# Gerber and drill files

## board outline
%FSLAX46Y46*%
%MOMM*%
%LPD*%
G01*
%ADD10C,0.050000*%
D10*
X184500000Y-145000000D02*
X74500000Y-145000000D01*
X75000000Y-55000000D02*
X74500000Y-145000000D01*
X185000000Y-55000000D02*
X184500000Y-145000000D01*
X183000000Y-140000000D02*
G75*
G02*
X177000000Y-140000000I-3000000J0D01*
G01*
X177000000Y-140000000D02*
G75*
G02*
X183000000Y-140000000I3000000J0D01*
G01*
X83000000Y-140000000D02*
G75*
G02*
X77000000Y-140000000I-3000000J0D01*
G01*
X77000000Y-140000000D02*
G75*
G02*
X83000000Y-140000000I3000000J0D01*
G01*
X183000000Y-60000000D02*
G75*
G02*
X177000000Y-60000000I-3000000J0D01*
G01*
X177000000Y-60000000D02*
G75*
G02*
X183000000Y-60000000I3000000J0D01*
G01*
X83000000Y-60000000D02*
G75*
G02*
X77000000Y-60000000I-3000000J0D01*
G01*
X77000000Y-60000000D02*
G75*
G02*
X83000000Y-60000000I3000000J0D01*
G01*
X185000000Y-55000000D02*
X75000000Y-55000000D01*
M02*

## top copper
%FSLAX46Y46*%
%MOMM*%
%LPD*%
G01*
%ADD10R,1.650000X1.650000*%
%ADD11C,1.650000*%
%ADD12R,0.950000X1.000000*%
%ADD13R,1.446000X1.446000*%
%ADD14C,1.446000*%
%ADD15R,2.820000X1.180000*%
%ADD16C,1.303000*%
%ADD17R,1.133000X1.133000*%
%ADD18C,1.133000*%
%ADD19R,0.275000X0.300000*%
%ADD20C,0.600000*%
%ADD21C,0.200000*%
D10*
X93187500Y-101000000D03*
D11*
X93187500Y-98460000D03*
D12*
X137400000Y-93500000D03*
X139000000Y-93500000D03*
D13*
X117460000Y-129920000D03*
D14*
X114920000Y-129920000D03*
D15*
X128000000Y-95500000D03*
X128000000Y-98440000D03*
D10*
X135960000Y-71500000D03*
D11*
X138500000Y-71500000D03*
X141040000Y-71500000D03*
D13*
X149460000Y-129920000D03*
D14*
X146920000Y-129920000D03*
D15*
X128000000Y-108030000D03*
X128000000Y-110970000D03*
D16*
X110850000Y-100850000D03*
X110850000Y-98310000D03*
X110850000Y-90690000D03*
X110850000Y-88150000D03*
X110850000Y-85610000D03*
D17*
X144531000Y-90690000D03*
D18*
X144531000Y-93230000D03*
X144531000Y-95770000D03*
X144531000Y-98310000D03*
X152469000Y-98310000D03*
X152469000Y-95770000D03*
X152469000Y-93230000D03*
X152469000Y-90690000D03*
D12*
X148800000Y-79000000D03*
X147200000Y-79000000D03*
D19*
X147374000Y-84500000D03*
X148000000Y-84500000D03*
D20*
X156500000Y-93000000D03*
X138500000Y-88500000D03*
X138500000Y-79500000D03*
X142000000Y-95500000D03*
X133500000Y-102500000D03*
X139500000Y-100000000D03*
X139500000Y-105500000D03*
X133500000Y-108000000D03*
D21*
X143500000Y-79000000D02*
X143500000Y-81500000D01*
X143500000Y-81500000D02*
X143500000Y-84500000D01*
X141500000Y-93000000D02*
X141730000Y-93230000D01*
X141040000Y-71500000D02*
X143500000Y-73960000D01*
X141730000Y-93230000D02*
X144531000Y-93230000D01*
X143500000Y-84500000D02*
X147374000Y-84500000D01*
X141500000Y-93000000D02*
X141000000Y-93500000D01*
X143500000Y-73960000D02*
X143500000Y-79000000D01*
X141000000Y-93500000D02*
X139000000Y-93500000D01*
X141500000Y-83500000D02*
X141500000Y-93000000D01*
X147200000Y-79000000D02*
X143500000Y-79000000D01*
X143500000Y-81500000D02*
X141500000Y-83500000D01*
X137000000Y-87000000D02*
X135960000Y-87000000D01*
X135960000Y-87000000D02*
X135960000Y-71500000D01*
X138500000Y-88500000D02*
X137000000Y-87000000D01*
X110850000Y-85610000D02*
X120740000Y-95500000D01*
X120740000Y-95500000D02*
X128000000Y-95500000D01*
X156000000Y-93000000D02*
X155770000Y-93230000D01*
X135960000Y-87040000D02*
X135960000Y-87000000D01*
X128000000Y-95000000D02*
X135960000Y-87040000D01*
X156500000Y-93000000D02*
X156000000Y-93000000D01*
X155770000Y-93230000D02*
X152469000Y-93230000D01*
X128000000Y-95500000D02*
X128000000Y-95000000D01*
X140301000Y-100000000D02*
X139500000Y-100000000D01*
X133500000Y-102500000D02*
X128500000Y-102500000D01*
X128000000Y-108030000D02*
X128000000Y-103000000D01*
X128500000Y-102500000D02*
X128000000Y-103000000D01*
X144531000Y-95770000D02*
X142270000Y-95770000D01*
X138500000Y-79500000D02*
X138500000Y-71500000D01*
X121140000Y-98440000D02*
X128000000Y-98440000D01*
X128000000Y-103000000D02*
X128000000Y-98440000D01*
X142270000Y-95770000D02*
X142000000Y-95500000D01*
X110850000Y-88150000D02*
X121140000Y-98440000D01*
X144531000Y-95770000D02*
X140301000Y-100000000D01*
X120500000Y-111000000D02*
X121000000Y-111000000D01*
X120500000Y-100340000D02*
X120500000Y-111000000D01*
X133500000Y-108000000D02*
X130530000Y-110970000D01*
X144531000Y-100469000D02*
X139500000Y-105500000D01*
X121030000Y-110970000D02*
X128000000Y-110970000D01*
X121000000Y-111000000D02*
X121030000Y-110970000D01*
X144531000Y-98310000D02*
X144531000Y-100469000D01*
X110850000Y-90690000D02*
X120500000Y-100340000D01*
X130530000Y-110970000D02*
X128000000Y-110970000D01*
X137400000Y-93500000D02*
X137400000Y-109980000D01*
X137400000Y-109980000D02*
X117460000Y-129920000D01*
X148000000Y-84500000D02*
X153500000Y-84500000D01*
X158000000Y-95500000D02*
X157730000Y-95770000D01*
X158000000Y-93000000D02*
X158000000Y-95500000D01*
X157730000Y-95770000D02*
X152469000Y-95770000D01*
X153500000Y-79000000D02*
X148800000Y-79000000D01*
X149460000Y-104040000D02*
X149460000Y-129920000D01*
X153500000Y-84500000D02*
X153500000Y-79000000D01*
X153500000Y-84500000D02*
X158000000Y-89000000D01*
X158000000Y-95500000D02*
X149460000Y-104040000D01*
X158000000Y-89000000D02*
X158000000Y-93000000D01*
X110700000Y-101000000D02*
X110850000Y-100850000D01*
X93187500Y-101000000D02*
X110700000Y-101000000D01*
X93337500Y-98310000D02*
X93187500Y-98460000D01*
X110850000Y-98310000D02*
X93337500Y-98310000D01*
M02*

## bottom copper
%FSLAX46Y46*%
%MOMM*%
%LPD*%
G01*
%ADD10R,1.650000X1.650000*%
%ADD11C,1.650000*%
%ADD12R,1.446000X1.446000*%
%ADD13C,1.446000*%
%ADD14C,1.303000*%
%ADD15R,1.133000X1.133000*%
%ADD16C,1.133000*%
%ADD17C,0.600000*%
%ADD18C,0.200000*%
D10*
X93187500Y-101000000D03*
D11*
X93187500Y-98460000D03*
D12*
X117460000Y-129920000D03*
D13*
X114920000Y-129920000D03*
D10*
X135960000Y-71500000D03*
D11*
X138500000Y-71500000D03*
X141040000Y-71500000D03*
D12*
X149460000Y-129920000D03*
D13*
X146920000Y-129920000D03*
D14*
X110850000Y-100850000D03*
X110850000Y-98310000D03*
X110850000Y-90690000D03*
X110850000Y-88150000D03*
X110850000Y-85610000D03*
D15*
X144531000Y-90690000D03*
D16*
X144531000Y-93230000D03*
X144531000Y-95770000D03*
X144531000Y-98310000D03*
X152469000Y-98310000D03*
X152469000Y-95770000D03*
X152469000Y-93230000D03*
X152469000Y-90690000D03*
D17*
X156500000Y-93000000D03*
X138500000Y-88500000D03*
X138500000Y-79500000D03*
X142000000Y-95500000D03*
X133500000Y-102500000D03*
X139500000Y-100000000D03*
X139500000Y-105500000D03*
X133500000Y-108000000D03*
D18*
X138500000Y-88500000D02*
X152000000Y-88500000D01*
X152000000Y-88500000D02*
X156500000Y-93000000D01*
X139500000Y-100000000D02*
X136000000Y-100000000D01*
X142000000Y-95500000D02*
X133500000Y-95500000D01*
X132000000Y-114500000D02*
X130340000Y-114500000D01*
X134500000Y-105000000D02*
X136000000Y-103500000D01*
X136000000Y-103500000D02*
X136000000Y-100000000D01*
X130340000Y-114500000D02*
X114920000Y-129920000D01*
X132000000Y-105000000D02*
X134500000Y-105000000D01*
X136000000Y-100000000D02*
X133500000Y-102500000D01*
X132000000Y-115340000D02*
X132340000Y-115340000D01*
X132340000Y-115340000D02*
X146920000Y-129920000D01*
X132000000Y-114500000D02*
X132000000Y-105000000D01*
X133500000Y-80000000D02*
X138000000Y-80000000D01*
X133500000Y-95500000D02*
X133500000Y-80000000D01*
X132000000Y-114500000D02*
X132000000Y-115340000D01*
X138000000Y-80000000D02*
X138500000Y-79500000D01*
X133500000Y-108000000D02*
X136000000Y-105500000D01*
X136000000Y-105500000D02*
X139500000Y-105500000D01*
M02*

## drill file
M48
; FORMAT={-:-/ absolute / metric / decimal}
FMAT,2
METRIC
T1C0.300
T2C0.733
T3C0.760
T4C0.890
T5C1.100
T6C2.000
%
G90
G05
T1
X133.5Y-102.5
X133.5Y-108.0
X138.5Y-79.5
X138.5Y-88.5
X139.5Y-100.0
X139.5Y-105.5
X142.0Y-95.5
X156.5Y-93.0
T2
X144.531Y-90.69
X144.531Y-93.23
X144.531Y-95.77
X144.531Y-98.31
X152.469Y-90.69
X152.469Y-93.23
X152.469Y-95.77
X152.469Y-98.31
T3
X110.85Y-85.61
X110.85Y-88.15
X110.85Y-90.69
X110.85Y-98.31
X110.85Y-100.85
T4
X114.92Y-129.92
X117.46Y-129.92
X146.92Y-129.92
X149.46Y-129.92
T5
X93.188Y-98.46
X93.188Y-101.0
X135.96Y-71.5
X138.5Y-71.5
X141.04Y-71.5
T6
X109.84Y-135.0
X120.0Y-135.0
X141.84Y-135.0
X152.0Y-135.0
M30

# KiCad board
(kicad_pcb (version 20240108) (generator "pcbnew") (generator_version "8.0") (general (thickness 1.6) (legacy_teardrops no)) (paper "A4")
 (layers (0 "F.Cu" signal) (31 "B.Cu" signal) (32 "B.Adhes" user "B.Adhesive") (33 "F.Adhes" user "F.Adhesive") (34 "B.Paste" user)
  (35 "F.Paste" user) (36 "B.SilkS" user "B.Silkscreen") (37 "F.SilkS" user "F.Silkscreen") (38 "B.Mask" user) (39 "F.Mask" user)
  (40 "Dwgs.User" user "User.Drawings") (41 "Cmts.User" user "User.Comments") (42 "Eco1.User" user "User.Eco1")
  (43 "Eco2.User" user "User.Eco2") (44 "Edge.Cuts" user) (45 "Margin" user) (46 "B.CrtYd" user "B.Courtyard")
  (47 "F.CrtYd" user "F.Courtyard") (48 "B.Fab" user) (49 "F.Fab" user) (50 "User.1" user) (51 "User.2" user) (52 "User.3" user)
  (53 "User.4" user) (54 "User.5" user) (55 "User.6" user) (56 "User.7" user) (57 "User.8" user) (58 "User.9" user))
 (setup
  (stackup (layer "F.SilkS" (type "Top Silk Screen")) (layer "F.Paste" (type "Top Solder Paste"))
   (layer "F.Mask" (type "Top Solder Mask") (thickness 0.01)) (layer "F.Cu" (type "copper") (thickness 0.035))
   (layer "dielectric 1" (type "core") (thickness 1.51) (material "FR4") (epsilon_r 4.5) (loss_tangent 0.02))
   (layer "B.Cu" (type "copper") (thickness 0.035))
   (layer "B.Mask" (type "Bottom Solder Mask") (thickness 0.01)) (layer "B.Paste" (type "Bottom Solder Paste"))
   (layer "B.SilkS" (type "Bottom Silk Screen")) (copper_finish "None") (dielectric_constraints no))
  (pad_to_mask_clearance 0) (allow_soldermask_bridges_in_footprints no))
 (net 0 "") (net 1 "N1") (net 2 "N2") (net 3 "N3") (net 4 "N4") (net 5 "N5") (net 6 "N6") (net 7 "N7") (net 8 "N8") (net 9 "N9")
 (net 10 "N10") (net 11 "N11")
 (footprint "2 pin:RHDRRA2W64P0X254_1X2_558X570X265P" (layer "F.Cu") (at 93.1875 101 90)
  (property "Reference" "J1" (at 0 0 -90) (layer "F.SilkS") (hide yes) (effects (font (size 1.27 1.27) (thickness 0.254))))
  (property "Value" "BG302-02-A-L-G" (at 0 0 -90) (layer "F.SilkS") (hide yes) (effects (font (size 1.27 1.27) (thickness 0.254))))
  (pad "1" thru_hole rect (at 0 0 90) (size 1.65 1.65) (drill 1.1) (layers "*.Cu" "*.Mask") (remove_unused_layers no) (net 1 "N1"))
  (pad "2" thru_hole circle (at 2.54 0 90) (size 1.65 1.65) (drill 1.1) (layers "*.Cu" "*.Mask") (remove_unused_layers no) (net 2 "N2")))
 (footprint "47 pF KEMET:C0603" (layer "F.Cu") (at 138.2 93.5)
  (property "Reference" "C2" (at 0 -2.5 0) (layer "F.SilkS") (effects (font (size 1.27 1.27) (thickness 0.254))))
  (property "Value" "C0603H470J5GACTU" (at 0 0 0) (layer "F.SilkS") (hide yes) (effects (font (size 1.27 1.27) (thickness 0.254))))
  (pad "1" smd rect (at -0.8 0) (size 0.95 1) (layers "F.Cu" "F.Paste" "F.Mask") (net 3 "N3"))
  (pad "2" smd rect (at 0.8 0) (size 0.95 1) (layers "F.Cu" "F.Paste" "F.Mask") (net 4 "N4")))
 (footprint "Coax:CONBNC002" (layer "F.Cu") (at 117.46 129.92)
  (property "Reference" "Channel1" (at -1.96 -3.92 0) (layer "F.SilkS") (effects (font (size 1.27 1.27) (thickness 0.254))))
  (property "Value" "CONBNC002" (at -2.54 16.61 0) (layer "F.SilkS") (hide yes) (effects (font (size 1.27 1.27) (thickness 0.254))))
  (pad "" np_thru_hole circle (at -7.62 5.08) (size 2 2) (drill 2) (layers "*.Cu" "*.Mask"))
  (pad "" np_thru_hole circle (at 2.54 5.08) (size 2 2) (drill 2) (layers "*.Cu" "*.Mask"))
  (pad "1" thru_hole rect (at 0 0) (size 1.446 1.446) (drill 0.89) (layers "*.Cu" "*.Mask") (remove_unused_layers no) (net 3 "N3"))
  (pad "2" thru_hole circle (at -2.54 0) (size 1.446 1.446) (drill 0.89) (layers "*.Cu" "*.Mask") (remove_unused_layers no) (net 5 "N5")))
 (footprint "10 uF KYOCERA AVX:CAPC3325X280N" (layer "F.Cu") (at 128 96.97 -90)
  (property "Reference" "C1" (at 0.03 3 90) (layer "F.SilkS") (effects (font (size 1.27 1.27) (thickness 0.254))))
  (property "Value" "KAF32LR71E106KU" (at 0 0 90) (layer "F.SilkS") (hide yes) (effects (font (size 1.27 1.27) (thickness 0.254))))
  (pad "1" smd rect (at -1.47 0 270) (size 1.18 2.82) (layers "F.Cu" "F.Paste" "F.Mask") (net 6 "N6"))
  (pad "2" smd rect (at 1.47 0 270) (size 1.18 2.82) (layers "F.Cu" "F.Paste" "F.Mask") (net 5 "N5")))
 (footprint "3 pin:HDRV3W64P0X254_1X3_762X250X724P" (layer "F.Cu") (at 135.96 71.5)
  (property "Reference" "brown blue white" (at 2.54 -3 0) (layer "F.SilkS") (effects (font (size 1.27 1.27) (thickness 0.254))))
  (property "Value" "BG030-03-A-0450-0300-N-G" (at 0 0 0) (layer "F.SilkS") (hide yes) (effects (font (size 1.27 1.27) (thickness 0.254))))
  (pad "1" thru_hole rect (at 0 0) (size 1.65 1.65) (drill 1.1) (layers "*.Cu" "*.Mask") (remove_unused_layers no) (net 6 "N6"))
  (pad "2" thru_hole circle (at 2.54 0) (size 1.65 1.65) (drill 1.1) (layers "*.Cu" "*.Mask") (remove_unused_layers no) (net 5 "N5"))
  (pad "3" thru_hole circle (at 5.08 0) (size 1.65 1.65) (drill 1.1) (layers "*.Cu" "*.Mask") (remove_unused_layers no) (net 4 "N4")))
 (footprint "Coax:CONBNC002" (layer "F.Cu") (at 149.46 129.92)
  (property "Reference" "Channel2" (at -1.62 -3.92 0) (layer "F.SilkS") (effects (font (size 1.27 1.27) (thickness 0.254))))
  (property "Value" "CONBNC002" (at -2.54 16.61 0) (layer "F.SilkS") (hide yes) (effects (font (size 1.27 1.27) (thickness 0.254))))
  (pad "" np_thru_hole circle (at -7.62 5.08) (size 2 2) (drill 2) (layers "*.Cu" "*.Mask"))
  (pad "" np_thru_hole circle (at 2.54 5.08) (size 2 2) (drill 2) (layers "*.Cu" "*.Mask"))
  (pad "1" thru_hole rect (at 0 0) (size 1.446 1.446) (drill 0.89) (layers "*.Cu" "*.Mask") (remove_unused_layers no) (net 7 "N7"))
  (pad "2" thru_hole circle (at -2.54 0) (size 1.446 1.446) (drill 0.89) (layers "*.Cu" "*.Mask") (remove_unused_layers no) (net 5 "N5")))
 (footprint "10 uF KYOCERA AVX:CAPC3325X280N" (layer "F.Cu") (at 128 109.5 -90)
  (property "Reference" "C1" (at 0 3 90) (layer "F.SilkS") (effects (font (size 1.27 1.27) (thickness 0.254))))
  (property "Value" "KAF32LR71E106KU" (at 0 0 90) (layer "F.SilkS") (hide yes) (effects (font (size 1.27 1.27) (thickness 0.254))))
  (pad "1" smd rect (at -1.47 0 270) (size 1.18 2.82) (layers "F.Cu" "F.Paste" "F.Mask") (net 5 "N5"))
  (pad "2" smd rect (at 1.47 0 270) (size 1.18 2.82) (layers "F.Cu" "F.Paste" "F.Mask") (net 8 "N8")))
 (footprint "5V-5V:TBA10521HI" (layer "F.Cu") (at 110.85 100.85 90)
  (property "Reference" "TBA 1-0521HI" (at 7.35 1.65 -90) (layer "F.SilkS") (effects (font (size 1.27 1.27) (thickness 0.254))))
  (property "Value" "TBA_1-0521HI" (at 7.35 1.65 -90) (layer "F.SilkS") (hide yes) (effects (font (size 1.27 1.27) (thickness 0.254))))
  (pad "1" thru_hole circle (at 0 0 90) (size 1.303 1.303) (drill 0.76) (layers "*.Cu" "*.Mask") (remove_unused_layers no) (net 1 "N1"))
  (pad "2" thru_hole circle (at 2.54 0 90) (size 1.303 1.303) (drill 0.76) (layers "*.Cu" "*.Mask") (remove_unused_layers no) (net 2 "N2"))
  (pad "5" thru_hole circle (at 10.16 0 90) (size 1.303 1.303) (drill 0.76) (layers "*.Cu" "*.Mask") (remove_unused_layers no) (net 8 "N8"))
  (pad "6" thru_hole circle (at 12.7 0 90) (size 1.303 1.303) (drill 0.76) (layers "*.Cu" "*.Mask") (remove_unused_layers no) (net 5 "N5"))
  (pad "7" thru_hole circle (at 15.24 0 90) (size 1.303 1.303) (drill 0.76) (layers "*.Cu" "*.Mask") (remove_unused_layers no) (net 6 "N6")))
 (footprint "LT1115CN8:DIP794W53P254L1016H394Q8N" (layer "F.Cu") (at 148.5 94.5)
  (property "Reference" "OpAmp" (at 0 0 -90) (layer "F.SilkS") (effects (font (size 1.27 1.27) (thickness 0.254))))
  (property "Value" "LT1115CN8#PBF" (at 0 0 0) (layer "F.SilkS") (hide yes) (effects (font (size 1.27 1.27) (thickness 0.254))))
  (pad "1" thru_hole rect (at -3.969 -3.81) (size 1.133 1.133) (drill 0.733) (layers "*.Cu" "*.Mask") (remove_unused_layers no) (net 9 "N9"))
  (pad "2" thru_hole circle (at -3.969 -1.27) (size 1.133 1.133) (drill 0.733) (layers "*.Cu" "*.Mask") (remove_unused_layers no)
   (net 4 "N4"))
  (pad "3" thru_hole circle (at -3.969 1.27) (size 1.133 1.133) (drill 0.733) (layers "*.Cu" "*.Mask") (remove_unused_layers no)
   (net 5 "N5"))
  (pad "4" thru_hole circle (at -3.969 3.81) (size 1.133 1.133) (drill 0.733) (layers "*.Cu" "*.Mask") (remove_unused_layers no)
   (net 8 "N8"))
  (pad "5" thru_hole circle (at 3.969 3.81) (size 1.133 1.133) (drill 0.733) (layers "*.Cu" "*.Mask") (remove_unused_layers no)
   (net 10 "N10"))
  (pad "6" thru_hole circle (at 3.969 1.27) (size 1.133 1.133) (drill 0.733) (layers "*.Cu" "*.Mask") (remove_unused_layers no) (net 7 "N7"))
  (pad "7" thru_hole circle (at 3.969 -1.27) (size 1.133 1.133) (drill 0.733) (layers "*.Cu" "*.Mask") (remove_unused_layers no)
   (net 6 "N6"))
  (pad "8" thru_hole circle (at 3.969 -3.81) (size 1.133 1.133) (drill 0.733) (layers "*.Cu" "*.Mask") (remove_unused_layers no)
   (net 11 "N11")))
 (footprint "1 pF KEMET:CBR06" (layer "F.Cu") (at 148 79 180)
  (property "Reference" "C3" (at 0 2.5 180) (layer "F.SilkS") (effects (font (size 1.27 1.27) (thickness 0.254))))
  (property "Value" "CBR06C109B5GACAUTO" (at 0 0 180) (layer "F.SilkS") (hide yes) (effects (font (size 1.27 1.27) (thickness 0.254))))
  (pad "1" smd rect (at -0.8 0 180) (size 0.95 1) (layers "F.Cu" "F.Paste" "F.Mask") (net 7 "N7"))
  (pad "2" smd rect (at 0.8 0 180) (size 0.95 1) (layers "F.Cu" "F.Paste" "F.Mask") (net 4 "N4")))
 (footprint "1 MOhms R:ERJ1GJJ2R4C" (layer "F.Cu") (at 147.687 84.5)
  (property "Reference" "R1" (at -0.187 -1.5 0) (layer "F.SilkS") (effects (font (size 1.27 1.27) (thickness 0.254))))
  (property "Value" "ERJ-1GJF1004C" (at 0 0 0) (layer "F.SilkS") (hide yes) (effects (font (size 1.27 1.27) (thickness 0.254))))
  (pad "1" smd rect (at -0.313 0) (size 0.275 0.3) (layers "F.Cu" "F.Paste" "F.Mask") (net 4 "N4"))
  (pad "2" smd rect (at 0.313 0) (size 0.275 0.3) (layers "F.Cu" "F.Paste" "F.Mask") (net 7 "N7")))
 (gr_line (start 184.5 145) (end 74.5 145) (stroke (width 0.05) (type default)) (layer "Edge.Cuts"))
 (gr_line (start 75 55) (end 74.5 145) (stroke (width 0.05) (type default)) (layer "Edge.Cuts"))
 (gr_line (start 185 55) (end 184.5 145) (stroke (width 0.05) (type default)) (layer "Edge.Cuts"))
 (gr_circle (center 180 140) (end 183 140) (stroke (width 0.05) (type default)) (fill none) (layer "Edge.Cuts"))
 (gr_circle (center 80 140) (end 83 140) (stroke (width 0.05) (type default)) (fill none) (layer "Edge.Cuts"))
 (gr_circle (center 180 60) (end 183 60) (stroke (width 0.05) (type default)) (fill none) (layer "Edge.Cuts"))
 (gr_circle (center 80 60) (end 83 60) (stroke (width 0.05) (type default)) (fill none) (layer "Edge.Cuts"))
 (gr_line (start 185 55) (end 75 55) (stroke (width 0.05) (type default)) (layer "Edge.Cuts"))
 (segment (start 143.5 79) (end 143.5 81.5) (width 0.2) (layer "F.Cu") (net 4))
 (segment (start 143.5 81.5) (end 143.5 84.5) (width 0.2) (layer "F.Cu") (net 4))
 (segment (start 141.5 93) (end 141.73 93.23) (width 0.2) (layer "F.Cu") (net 4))
 (segment (start 141.04 71.5) (end 143.5 73.96) (width 0.2) (layer "F.Cu") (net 4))
 (segment (start 141.73 93.23) (end 144.531 93.23) (width 0.2) (layer "F.Cu") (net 4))
 (segment (start 143.5 84.5) (end 147.374 84.5) (width 0.2) (layer "F.Cu") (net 4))
 (segment (start 141.5 93) (end 141 93.5) (width 0.2) (layer "F.Cu") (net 4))
 (segment (start 143.5 73.96) (end 143.5 79) (width 0.2) (layer "F.Cu") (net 4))
 (segment (start 141 93.5) (end 139 93.5) (width 0.2) (layer "F.Cu") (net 4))
 (segment (start 141.5 83.5) (end 141.5 93) (width 0.2) (layer "F.Cu") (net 4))
 (segment (start 147.2 79) (end 143.5 79) (width 0.2) (layer "F.Cu") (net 4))
 (segment (start 143.5 81.5) (end 141.5 83.5) (width 0.2) (layer "F.Cu") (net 4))
 (segment (start 137 87) (end 135.96 87) (width 0.2) (layer "F.Cu") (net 6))
 (segment (start 135.96 87) (end 135.96 71.5) (width 0.2) (layer "F.Cu") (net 6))
 (segment (start 138.5 88.5) (end 137 87) (width 0.2) (layer "F.Cu") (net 6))
 (segment (start 110.85 85.61) (end 120.74 95.5) (width 0.2) (layer "F.Cu") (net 6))
 (segment (start 120.74 95.5) (end 128 95.5) (width 0.2) (layer "F.Cu") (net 6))
 (segment (start 156 93) (end 155.77 93.23) (width 0.2) (layer "F.Cu") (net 6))
 (segment (start 135.96 87.04) (end 135.96 87) (width 0.2) (layer "F.Cu") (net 6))
 (segment (start 128 95) (end 135.96 87.04) (width 0.2) (layer "F.Cu") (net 6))
 (segment (start 156.5 93) (end 156 93) (width 0.2) (layer "F.Cu") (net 6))
 (segment (start 155.77 93.23) (end 152.469 93.23) (width 0.2) (layer "F.Cu") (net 6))
 (segment (start 128 95.5) (end 128 95) (width 0.2) (layer "F.Cu") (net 6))
 (via (at 156.5 93) (size 0.6) (drill 0.3) (layers "F.Cu" "B.Cu") (free yes) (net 6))
 (via (at 138.5 88.5) (size 0.6) (drill 0.3) (layers "F.Cu" "B.Cu") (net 6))
 (segment (start 138.5 88.5) (end 152 88.5) (width 0.2) (layer "B.Cu") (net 6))
 (segment (start 152 88.5) (end 156.5 93) (width 0.2) (layer "B.Cu") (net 6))
 (segment (start 140.301 100) (end 139.5 100) (width 0.2) (layer "F.Cu") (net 5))
 (segment (start 133.5 102.5) (end 128.5 102.5) (width 0.2) (layer "F.Cu") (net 5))
 (segment (start 128 108.03) (end 128 103) (width 0.2) (layer "F.Cu") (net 5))
 (segment (start 128.5 102.5) (end 128 103) (width 0.2) (layer "F.Cu") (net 5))
 (segment (start 144.531 95.77) (end 142.27 95.77) (width 0.2) (layer "F.Cu") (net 5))
 (segment (start 138.5 79.5) (end 138.5 71.5) (width 0.2) (layer "F.Cu") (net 5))
 (segment (start 121.14 98.44) (end 128 98.44) (width 0.2) (layer "F.Cu") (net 5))
 (segment (start 128 103) (end 128 98.44) (width 0.2) (layer "F.Cu") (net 5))
 (segment (start 142.27 95.77) (end 142 95.5) (width 0.2) (layer "F.Cu") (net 5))
 (segment (start 110.85 88.15) (end 121.14 98.44) (width 0.2) (layer "F.Cu") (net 5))
 (segment (start 144.531 95.77) (end 140.301 100) (width 0.2) (layer "F.Cu") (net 5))
 (via (at 138.5 79.5) (size 0.6) (drill 0.3) (layers "F.Cu" "B.Cu") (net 5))
 (via (at 142 95.5) (size 0.6) (drill 0.3) (layers "F.Cu" "B.Cu") (free yes) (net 5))
 (via (at 133.5 102.5) (size 0.6) (drill 0.3) (layers "F.Cu" "B.Cu") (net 5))
 (via (at 139.5 100) (size 0.6) (drill 0.3) (layers "F.Cu" "B.Cu") (free yes) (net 5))
 (segment (start 139.5 100) (end 136 100) (width 0.2) (layer "B.Cu") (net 5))
 (segment (start 142 95.5) (end 133.5 95.5) (width 0.2) (layer "B.Cu") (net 5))
 (segment (start 132 114.5) (end 130.34 114.5) (width 0.2) (layer "B.Cu") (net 5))
 (segment (start 134.5 105) (end 136 103.5) (width 0.2) (layer "B.Cu") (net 5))
 (segment (start 136 103.5) (end 136 100) (width 0.2) (layer "B.Cu") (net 5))
 (segment (start 130.34 114.5) (end 114.92 129.92) (width 0.2) (layer "B.Cu") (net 5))
 (segment (start 132 105) (end 134.5 105) (width 0.2) (layer "B.Cu") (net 5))
 (segment (start 136 100) (end 133.5 102.5) (width 0.2) (layer "B.Cu") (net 5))
 (segment (start 132 115.34) (end 132.34 115.34) (width 0.2) (layer "B.Cu") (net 5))
 (segment (start 132.34 115.34) (end 146.92 129.92) (width 0.2) (layer "B.Cu") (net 5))
 (segment (start 132 114.5) (end 132 105) (width 0.2) (layer "B.Cu") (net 5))
 (segment (start 133.5 80) (end 138 80) (width 0.2) (layer "B.Cu") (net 5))
 (segment (start 133.5 95.5) (end 133.5 80) (width 0.2) (layer "B.Cu") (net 5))
 (segment (start 132 114.5) (end 132 115.34) (width 0.2) (layer "B.Cu") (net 5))
 (segment (start 138 80) (end 138.5 79.5) (width 0.2) (layer "B.Cu") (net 5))
 (segment (start 120.5 111) (end 121 111) (width 0.2) (layer "F.Cu") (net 8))
 (segment (start 120.5 100.34) (end 120.5 111) (width 0.2) (layer "F.Cu") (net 8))
 (segment (start 133.5 108) (end 130.53 110.97) (width 0.2) (layer "F.Cu") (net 8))
 (segment (start 144.531 100.469) (end 139.5 105.5) (width 0.2) (layer "F.Cu") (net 8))
 (segment (start 121.03 110.97) (end 128 110.97) (width 0.2) (layer "F.Cu") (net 8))
 (segment (start 121 111) (end 121.03 110.97) (width 0.2) (layer "F.Cu") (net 8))
 (segment (start 144.531 98.31) (end 144.531 100.469) (width 0.2) (layer "F.Cu") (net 8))
 (segment (start 110.85 90.69) (end 120.5 100.34) (width 0.2) (layer "F.Cu") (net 8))
 (segment (start 130.53 110.97) (end 128 110.97) (width 0.2) (layer "F.Cu") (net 8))
 (via (at 139.5 105.5) (size 0.6) (drill 0.3) (layers "F.Cu" "B.Cu") (free yes) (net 8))
 (via (at 133.5 108) (size 0.6) (drill 0.3) (layers "F.Cu" "B.Cu") (free yes) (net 8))
 (segment (start 133.5 108) (end 136 105.5) (width 0.2) (layer "B.Cu") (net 8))
 (segment (start 136 105.5) (end 139.5 105.5) (width 0.2) (layer "B.Cu") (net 8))
 (segment (start 137.4 93.5) (end 137.4 109.98) (width 0.2) (layer "F.Cu") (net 3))
 (segment (start 137.4 109.98) (end 117.46 129.92) (width 0.2) (layer "F.Cu") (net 3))
 (segment (start 148 84.5) (end 153.5 84.5) (width 0.2) (layer "F.Cu") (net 7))
 (segment (start 158 95.5) (end 157.73 95.77) (width 0.2) (layer "F.Cu") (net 7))
 (segment (start 158 93) (end 158 95.5) (width 0.2) (layer "F.Cu") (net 7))
 (segment (start 157.73 95.77) (end 152.469 95.77) (width 0.2) (layer "F.Cu") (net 7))
 (segment (start 153.5 79) (end 148.8 79) (width 0.2) (layer "F.Cu") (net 7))
 (segment (start 149.46 104.04) (end 149.46 129.92) (width 0.2) (layer "F.Cu") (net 7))
 (segment (start 153.5 84.5) (end 153.5 79) (width 0.2) (layer "F.Cu") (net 7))
 (segment (start 153.5 84.5) (end 158 89) (width 0.2) (layer "F.Cu") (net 7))
 (segment (start 158 95.5) (end 149.46 104.04) (width 0.2) (layer "F.Cu") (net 7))
 (segment (start 158 89) (end 158 93) (width 0.2) (layer "F.Cu") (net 7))
 (segment (start 110.7 101) (end 110.85 100.85) (width 0.2) (layer "F.Cu") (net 1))
 (segment (start 93.1875 101) (end 110.7 101) (width 0.2) (layer "F.Cu") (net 1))
 (segment (start 93.3375 98.31) (end 93.1875 98.46) (width 0.2) (layer "F.Cu") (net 2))
 (segment (start 110.85 98.31) (end 93.3375 98.31) (width 0.2) (layer "F.Cu") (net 2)))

